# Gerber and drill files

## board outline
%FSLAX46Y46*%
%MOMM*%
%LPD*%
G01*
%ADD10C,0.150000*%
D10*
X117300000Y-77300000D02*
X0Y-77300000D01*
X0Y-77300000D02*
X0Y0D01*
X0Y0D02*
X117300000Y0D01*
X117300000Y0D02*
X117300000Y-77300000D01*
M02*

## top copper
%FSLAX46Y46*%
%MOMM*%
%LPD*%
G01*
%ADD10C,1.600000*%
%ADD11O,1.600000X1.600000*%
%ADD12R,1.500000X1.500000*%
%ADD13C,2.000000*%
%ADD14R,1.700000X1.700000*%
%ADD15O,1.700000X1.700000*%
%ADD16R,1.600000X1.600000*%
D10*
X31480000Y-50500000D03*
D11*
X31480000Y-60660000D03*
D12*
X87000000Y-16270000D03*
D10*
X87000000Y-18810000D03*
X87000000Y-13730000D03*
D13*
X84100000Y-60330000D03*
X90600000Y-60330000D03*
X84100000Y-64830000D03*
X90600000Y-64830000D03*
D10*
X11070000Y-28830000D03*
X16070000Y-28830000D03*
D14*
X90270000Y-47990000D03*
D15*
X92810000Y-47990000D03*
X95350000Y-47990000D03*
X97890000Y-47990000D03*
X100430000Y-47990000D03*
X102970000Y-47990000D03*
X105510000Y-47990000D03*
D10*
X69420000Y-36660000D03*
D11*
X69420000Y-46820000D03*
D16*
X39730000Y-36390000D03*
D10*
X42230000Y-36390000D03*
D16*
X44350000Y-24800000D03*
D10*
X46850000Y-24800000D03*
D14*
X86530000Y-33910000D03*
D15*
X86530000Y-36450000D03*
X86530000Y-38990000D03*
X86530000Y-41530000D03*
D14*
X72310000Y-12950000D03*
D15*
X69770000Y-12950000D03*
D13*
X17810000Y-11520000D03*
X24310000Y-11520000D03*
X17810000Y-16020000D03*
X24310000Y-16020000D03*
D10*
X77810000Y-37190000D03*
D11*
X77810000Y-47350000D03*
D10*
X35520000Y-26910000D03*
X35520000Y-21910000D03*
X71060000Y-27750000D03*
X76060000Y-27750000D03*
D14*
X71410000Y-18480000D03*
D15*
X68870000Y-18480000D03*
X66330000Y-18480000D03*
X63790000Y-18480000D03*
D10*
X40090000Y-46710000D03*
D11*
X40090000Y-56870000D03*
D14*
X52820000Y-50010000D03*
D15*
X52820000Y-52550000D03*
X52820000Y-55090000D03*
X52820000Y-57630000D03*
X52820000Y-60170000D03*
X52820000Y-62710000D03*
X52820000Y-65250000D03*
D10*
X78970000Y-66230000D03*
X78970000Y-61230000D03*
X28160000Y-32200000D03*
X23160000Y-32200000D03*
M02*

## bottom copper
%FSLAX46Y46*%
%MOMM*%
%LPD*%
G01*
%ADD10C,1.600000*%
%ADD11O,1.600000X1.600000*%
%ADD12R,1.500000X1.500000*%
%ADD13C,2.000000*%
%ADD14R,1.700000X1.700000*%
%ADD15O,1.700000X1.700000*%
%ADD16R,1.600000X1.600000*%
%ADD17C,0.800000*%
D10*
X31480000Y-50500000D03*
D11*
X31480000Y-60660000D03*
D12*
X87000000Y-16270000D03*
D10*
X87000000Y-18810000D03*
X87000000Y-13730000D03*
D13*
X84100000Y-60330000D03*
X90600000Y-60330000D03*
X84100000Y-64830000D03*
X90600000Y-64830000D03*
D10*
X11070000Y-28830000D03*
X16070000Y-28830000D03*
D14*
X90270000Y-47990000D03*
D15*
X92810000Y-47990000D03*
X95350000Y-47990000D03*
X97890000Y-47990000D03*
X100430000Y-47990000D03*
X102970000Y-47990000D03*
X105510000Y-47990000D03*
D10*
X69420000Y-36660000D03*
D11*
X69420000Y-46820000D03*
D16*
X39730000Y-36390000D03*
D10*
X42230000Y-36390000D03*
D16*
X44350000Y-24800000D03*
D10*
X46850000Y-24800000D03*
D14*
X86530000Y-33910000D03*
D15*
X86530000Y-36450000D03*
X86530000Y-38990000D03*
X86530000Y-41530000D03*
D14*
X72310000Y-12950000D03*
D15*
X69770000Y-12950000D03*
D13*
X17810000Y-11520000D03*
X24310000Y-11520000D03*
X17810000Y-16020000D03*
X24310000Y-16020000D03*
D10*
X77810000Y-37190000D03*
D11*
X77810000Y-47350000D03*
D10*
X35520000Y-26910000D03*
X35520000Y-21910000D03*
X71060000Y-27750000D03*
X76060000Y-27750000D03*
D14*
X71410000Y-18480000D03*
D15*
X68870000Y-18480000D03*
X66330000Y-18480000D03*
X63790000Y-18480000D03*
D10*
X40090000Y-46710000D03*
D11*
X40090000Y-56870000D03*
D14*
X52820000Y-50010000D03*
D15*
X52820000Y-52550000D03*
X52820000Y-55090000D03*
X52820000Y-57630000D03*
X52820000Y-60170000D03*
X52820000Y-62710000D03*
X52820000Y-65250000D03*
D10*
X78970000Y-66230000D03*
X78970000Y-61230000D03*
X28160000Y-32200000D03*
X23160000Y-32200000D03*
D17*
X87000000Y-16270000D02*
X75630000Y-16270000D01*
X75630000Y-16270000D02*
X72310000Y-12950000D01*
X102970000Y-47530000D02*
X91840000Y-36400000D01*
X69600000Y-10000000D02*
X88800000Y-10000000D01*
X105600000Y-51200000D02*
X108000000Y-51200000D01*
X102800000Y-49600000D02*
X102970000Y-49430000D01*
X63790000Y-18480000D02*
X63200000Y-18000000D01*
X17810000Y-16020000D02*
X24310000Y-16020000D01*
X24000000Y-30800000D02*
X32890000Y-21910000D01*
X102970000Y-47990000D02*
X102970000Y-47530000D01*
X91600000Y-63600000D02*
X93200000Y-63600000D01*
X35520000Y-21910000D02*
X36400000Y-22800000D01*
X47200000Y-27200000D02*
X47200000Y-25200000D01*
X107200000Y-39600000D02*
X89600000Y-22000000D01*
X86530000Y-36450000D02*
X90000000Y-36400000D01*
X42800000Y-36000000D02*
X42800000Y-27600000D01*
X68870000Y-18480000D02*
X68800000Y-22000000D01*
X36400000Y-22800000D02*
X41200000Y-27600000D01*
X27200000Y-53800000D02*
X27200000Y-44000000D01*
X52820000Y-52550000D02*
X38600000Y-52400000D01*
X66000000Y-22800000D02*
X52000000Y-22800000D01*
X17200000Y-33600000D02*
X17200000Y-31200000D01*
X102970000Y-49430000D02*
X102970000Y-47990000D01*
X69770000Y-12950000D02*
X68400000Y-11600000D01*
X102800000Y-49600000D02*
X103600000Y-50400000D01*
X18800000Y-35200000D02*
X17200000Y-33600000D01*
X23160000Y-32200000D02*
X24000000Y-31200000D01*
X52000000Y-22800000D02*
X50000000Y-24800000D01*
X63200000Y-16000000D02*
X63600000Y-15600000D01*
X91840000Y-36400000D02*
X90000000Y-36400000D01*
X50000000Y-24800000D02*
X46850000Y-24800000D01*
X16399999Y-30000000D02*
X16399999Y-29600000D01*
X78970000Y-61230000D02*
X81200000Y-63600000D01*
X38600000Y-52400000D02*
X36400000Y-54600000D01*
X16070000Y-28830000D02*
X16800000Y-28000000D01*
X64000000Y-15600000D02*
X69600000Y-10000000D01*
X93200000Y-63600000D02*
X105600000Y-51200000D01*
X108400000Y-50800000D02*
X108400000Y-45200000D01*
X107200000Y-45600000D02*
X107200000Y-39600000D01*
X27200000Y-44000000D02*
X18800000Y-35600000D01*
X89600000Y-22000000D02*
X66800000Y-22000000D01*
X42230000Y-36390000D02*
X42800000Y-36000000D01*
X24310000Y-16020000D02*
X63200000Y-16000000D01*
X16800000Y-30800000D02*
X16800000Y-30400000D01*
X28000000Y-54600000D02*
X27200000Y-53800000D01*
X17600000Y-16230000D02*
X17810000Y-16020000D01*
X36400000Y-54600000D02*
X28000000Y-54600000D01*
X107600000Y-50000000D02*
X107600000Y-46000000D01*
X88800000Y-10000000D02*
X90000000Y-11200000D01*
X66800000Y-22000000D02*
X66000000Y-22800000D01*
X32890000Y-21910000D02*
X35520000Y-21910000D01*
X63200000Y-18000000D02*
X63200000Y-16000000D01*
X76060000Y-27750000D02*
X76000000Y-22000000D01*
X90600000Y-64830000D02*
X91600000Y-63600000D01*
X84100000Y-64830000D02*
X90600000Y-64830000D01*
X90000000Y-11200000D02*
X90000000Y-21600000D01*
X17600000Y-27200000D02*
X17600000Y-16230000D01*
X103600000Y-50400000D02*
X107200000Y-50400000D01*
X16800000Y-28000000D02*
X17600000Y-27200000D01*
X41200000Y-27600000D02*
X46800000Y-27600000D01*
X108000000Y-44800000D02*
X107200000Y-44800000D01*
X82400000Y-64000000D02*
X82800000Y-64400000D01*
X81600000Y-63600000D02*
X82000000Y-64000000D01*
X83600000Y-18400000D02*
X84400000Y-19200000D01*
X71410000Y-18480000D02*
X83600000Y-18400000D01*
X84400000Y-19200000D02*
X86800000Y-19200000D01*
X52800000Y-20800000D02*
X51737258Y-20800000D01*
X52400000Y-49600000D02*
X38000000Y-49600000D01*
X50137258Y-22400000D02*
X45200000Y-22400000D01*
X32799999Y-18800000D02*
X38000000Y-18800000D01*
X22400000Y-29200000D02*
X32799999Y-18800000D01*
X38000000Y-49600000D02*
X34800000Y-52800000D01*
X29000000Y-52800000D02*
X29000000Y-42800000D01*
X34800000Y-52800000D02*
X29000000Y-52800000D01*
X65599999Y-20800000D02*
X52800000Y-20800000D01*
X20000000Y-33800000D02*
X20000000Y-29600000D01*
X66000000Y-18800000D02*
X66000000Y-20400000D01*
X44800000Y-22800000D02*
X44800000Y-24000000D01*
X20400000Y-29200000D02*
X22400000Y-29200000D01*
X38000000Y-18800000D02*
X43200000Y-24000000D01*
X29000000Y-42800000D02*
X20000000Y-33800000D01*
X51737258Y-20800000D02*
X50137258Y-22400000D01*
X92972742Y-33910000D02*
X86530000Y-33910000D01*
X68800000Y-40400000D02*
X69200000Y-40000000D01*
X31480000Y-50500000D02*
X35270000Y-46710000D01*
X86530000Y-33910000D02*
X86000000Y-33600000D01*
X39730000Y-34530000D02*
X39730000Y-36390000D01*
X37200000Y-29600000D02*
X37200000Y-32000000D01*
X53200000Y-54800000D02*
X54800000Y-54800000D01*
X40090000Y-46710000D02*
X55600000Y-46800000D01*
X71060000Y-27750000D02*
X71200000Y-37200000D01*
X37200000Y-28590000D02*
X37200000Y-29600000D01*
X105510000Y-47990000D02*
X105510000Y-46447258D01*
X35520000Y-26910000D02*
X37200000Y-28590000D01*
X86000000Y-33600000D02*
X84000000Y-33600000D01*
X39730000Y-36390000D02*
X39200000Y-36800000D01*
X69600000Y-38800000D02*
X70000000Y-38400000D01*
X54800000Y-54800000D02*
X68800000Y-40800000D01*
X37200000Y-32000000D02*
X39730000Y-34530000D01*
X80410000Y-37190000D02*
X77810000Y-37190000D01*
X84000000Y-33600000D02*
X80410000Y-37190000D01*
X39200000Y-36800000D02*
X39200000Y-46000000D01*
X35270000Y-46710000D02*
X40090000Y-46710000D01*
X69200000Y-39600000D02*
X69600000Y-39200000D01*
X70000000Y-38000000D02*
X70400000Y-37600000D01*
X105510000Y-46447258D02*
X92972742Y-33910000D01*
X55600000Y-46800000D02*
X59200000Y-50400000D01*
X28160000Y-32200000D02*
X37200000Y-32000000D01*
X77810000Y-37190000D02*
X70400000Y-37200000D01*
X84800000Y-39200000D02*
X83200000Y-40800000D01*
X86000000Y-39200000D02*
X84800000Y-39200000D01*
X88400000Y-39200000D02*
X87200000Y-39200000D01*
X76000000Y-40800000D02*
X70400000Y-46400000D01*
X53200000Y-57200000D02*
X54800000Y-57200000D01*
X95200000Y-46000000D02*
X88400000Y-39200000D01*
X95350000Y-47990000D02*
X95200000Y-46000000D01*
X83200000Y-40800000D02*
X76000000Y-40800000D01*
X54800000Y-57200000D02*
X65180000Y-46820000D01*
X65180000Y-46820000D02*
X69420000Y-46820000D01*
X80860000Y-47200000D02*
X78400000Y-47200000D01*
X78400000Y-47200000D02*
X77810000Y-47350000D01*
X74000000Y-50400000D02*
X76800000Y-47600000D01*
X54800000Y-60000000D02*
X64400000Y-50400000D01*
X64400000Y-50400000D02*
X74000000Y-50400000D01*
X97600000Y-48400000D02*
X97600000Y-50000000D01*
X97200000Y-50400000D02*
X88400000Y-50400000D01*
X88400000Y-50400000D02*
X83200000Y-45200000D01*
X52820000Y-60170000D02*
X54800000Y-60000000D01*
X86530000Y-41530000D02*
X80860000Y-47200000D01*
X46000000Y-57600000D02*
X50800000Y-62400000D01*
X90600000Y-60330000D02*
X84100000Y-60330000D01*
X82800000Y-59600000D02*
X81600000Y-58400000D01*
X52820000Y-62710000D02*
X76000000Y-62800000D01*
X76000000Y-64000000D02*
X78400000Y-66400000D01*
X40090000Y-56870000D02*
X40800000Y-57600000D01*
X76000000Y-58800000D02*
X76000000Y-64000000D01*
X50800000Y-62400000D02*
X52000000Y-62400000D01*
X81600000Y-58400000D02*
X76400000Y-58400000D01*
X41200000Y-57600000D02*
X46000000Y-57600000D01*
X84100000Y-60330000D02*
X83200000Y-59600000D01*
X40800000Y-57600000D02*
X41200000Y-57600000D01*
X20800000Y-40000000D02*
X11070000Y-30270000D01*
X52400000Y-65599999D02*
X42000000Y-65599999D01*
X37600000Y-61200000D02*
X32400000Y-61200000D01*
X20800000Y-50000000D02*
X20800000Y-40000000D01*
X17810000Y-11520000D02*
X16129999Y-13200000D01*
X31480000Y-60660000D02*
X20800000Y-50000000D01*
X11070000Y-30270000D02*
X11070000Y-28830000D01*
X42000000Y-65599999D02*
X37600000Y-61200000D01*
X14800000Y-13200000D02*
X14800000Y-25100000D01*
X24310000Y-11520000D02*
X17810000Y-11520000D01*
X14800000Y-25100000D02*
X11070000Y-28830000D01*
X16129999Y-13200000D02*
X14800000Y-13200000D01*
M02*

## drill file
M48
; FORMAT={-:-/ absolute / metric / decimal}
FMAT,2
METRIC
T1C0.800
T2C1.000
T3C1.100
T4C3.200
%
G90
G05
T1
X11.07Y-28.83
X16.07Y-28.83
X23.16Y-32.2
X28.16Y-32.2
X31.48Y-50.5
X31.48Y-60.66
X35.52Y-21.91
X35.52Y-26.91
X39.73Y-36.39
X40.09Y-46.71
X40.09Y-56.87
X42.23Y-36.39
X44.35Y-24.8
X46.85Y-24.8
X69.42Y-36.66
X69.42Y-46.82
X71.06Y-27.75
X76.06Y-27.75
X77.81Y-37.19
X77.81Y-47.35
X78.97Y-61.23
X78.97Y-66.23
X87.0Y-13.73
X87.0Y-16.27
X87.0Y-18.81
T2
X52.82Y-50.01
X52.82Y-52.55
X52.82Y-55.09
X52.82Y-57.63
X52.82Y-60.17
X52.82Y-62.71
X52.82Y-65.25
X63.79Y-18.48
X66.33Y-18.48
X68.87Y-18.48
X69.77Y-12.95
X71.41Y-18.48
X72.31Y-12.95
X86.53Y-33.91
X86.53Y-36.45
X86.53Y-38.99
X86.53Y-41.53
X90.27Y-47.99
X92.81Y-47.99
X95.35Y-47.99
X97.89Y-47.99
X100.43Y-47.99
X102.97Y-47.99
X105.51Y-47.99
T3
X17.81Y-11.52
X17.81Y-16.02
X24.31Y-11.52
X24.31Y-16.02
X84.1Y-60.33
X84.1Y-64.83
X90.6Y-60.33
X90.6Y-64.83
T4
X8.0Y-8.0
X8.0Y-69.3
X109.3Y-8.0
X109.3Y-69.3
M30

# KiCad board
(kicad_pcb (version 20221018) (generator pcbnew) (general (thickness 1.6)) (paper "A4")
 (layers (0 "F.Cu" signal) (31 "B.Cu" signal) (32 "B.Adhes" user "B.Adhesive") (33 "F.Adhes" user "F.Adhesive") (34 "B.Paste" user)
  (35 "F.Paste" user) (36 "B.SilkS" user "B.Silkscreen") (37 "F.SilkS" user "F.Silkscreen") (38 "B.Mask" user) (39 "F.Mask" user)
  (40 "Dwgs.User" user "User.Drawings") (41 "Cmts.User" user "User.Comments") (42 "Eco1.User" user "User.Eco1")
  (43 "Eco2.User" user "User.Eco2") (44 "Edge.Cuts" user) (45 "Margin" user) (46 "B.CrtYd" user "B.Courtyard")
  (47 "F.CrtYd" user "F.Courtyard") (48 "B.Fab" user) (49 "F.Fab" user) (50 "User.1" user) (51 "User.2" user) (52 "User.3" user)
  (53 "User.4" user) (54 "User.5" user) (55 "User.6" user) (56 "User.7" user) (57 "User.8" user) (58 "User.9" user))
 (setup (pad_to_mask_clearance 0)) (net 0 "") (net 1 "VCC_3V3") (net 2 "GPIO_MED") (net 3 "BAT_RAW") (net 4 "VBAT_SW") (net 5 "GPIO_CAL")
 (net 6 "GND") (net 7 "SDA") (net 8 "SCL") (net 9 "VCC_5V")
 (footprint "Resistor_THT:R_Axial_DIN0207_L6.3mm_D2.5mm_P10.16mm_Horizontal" (layer "F.Cu") (at 31.48 50.5 -90)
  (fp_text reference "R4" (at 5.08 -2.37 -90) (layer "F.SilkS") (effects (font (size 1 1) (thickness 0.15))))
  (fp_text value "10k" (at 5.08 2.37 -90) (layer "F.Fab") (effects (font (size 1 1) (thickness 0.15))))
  (pad "1" thru_hole circle (at 0 0 270) (size 1.6 1.6) (drill 0.8) (layers "*.Cu" "*.Mask") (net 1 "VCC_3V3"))
  (pad "2" thru_hole oval (at 10.16 0 270) (size 1.6 1.6) (drill 0.8) (layers "*.Cu" "*.Mask") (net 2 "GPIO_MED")))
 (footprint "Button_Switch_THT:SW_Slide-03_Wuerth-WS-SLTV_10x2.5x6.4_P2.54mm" (layer "F.Cu") (at 87 16.27 90)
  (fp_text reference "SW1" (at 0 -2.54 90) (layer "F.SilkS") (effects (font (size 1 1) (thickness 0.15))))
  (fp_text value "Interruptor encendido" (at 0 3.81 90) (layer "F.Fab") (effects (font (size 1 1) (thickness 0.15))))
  (pad "1" thru_hole rect (at 0 0 90) (size 1.5 1.5) (drill 0.8) (layers "*.Cu" "*.Mask") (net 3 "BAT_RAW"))
  (pad "2" thru_hole circle (at -2.54 0 90) (size 1.6 1.6) (drill 0.8) (layers "*.Cu" "*.Mask") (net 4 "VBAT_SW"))
  (pad "3" thru_hole circle (at 2.54 0 90) (size 1.6 1.6) (drill 0.8) (layers "*.Cu" "*.Mask")))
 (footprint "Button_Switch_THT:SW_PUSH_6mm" (layer "F.Cu") (at 84.1 60.33)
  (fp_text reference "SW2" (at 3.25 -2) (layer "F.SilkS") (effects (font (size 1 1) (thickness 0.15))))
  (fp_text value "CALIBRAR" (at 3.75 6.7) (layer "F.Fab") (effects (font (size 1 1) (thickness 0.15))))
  (pad "1" thru_hole circle (at 0 0 90) (size 2 2) (drill 1.1) (layers "*.Cu" "*.Mask") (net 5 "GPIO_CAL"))
  (pad "1" thru_hole circle (at 6.5 0 90) (size 2 2) (drill 1.1) (layers "*.Cu" "*.Mask") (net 5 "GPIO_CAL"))
  (pad "2" thru_hole circle (at 0 4.5 90) (size 2 2) (drill 1.1) (layers "*.Cu" "*.Mask") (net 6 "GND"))
  (pad "2" thru_hole circle (at 6.5 4.5 90) (size 2 2) (drill 1.1) (layers "*.Cu" "*.Mask") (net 6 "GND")))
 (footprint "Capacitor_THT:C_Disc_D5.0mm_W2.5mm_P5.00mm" (layer "F.Cu") (at 11.07 28.83)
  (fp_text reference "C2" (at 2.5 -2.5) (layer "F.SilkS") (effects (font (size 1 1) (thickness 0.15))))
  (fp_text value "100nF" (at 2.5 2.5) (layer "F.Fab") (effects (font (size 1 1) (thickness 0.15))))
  (pad "1" thru_hole circle (at 0 0) (size 1.6 1.6) (drill 0.8) (layers "*.Cu" "*.Mask") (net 2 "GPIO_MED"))
  (pad "2" thru_hole circle (at 5 0) (size 1.6 1.6) (drill 0.8) (layers "*.Cu" "*.Mask") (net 6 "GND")))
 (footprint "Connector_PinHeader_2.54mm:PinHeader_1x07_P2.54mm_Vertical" (layer "F.Cu") (at 90.27 47.99 90)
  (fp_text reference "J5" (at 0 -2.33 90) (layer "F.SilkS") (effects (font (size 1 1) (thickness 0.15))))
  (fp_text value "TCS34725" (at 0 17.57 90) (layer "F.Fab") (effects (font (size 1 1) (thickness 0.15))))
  (pad "1" thru_hole rect (at 0 0 90) (size 1.7 1.7) (drill 1) (layers "*.Cu" "*.Mask"))
  (pad "2" thru_hole oval (at 0 2.54 90) (size 1.7 1.7) (drill 1) (layers "*.Cu" "*.Mask"))
  (pad "3" thru_hole oval (at 0 5.08 90) (size 1.7 1.7) (drill 1) (layers "*.Cu" "*.Mask") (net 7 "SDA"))
  (pad "4" thru_hole oval (at 0 7.62 90) (size 1.7 1.7) (drill 1) (layers "*.Cu" "*.Mask") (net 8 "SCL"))
  (pad "5" thru_hole oval (at 0 10.16 90) (size 1.7 1.7) (drill 1) (layers "*.Cu" "*.Mask"))
  (pad "6" thru_hole oval (at 0 12.7 90) (size 1.7 1.7) (drill 1) (layers "*.Cu" "*.Mask") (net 6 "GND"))
  (pad "7" thru_hole oval (at 0 15.24 90) (size 1.7 1.7) (drill 1) (layers "*.Cu" "*.Mask") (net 1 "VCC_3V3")))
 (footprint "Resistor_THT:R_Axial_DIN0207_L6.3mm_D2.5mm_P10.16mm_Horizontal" (layer "F.Cu") (at 69.42 36.66 -90)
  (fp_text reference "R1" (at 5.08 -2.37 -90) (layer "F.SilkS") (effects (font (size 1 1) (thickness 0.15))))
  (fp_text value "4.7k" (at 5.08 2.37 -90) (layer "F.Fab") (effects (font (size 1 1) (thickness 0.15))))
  (pad "1" thru_hole circle (at 0 0 270) (size 1.6 1.6) (drill 0.8) (layers "*.Cu" "*.Mask") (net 1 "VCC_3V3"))
  (pad "2" thru_hole oval (at 10.16 0 270) (size 1.6 1.6) (drill 0.8) (layers "*.Cu" "*.Mask") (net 7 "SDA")))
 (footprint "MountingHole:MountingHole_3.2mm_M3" (layer "F.Cu") (at 8 69.3)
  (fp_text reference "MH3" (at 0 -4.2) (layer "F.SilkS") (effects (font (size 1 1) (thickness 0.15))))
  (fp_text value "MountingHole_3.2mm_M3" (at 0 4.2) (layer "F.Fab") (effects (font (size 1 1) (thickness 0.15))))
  (pad "" np_thru_hole circle (at 0 0) (size 3.2 3.2) (drill 3.2) (layers "*.Cu" "*.Mask")))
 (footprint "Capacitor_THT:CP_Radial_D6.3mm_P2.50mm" (layer "F.Cu") (at 39.73 36.39)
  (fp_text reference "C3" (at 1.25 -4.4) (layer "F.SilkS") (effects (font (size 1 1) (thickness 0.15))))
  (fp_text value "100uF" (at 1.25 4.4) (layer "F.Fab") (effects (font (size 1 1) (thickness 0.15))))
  (pad "1" thru_hole rect (at 0 0) (size 1.6 1.6) (drill 0.8) (layers "*.Cu" "*.Mask") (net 1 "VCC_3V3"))
  (pad "2" thru_hole circle (at 2.5 0) (size 1.6 1.6) (drill 0.8) (layers "*.Cu" "*.Mask") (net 6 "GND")))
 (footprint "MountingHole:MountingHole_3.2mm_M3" (layer "F.Cu") (at 109.3 8)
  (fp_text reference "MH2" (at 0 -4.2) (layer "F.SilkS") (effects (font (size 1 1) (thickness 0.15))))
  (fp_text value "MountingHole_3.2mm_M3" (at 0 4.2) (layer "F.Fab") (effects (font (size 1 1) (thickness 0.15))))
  (pad "" np_thru_hole circle (at 0 0) (size 3.2 3.2) (drill 3.2) (layers "*.Cu" "*.Mask")))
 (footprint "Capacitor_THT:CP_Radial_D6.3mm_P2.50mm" (layer "F.Cu") (at 44.35 24.8)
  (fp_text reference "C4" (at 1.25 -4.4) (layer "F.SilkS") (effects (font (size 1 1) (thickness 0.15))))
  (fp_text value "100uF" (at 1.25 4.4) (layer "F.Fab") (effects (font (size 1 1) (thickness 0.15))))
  (pad "1" thru_hole rect (at 0 0) (size 1.6 1.6) (drill 0.8) (layers "*.Cu" "*.Mask") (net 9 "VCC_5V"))
  (pad "2" thru_hole circle (at 2.5 0) (size 1.6 1.6) (drill 0.8) (layers "*.Cu" "*.Mask") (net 6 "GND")))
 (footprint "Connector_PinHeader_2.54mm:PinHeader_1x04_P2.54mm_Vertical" (layer "F.Cu") (at 86.53 33.91)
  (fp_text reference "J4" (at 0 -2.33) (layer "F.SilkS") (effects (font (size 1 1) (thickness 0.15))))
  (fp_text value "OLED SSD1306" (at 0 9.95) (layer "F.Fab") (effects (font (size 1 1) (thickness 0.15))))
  (pad "1" thru_hole rect (at 0 0) (size 1.7 1.7) (drill 1) (layers "*.Cu" "*.Mask") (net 1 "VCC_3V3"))
  (pad "2" thru_hole oval (at 0 2.54) (size 1.7 1.7) (drill 1) (layers "*.Cu" "*.Mask") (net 6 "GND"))
  (pad "3" thru_hole oval (at 0 5.08) (size 1.7 1.7) (drill 1) (layers "*.Cu" "*.Mask") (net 7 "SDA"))
  (pad "4" thru_hole oval (at 0 7.62) (size 1.7 1.7) (drill 1) (layers "*.Cu" "*.Mask") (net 8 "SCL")))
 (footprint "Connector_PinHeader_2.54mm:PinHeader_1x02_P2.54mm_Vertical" (layer "F.Cu") (at 72.31 12.95 -90)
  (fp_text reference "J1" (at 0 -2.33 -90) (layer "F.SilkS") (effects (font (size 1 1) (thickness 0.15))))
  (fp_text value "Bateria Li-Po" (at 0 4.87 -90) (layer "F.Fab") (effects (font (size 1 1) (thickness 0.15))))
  (pad "1" thru_hole rect (at 0 0 270) (size 1.7 1.7) (drill 1) (layers "*.Cu" "*.Mask") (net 3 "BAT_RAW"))
  (pad "2" thru_hole oval (at 0 2.54 270) (size 1.7 1.7) (drill 1) (layers "*.Cu" "*.Mask") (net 6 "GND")))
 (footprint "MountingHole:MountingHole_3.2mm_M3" (layer "F.Cu") (at 109.3 69.3)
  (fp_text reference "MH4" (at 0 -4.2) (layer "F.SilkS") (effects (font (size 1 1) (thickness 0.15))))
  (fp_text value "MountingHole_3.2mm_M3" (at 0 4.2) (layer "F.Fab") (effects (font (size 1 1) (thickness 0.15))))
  (pad "" np_thru_hole circle (at 0 0) (size 3.2 3.2) (drill 3.2) (layers "*.Cu" "*.Mask")))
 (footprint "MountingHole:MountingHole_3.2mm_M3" (layer "F.Cu") (at 8 8)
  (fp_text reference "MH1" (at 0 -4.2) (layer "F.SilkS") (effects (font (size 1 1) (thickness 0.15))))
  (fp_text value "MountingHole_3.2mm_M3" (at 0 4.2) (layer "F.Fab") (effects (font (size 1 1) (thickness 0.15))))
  (pad "" np_thru_hole circle (at 0 0) (size 3.2 3.2) (drill 3.2) (layers "*.Cu" "*.Mask")))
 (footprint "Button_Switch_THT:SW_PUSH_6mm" (layer "F.Cu") (at 17.81 11.52)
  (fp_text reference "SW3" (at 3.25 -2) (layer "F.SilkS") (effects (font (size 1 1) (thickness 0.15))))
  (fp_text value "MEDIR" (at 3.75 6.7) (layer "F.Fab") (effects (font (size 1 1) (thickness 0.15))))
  (pad "1" thru_hole circle (at 0 0 90) (size 2 2) (drill 1.1) (layers "*.Cu" "*.Mask") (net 2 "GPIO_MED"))
  (pad "1" thru_hole circle (at 6.5 0 90) (size 2 2) (drill 1.1) (layers "*.Cu" "*.Mask") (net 2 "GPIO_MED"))
  (pad "2" thru_hole circle (at 0 4.5 90) (size 2 2) (drill 1.1) (layers "*.Cu" "*.Mask") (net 6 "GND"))
  (pad "2" thru_hole circle (at 6.5 4.5 90) (size 2 2) (drill 1.1) (layers "*.Cu" "*.Mask") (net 6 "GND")))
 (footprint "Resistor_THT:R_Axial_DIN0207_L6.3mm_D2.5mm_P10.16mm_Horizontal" (layer "F.Cu") (at 77.81 37.19 -90)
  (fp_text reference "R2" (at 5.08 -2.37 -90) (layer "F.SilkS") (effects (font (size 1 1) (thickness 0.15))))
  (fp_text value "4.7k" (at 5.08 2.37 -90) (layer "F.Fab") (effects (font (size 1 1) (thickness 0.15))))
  (pad "1" thru_hole circle (at 0 0 270) (size 1.6 1.6) (drill 0.8) (layers "*.Cu" "*.Mask") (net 1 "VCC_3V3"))
  (pad "2" thru_hole oval (at 10.16 0 270) (size 1.6 1.6) (drill 0.8) (layers "*.Cu" "*.Mask") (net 8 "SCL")))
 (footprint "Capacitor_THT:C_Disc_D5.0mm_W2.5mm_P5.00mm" (layer "F.Cu") (at 35.52 26.91 90)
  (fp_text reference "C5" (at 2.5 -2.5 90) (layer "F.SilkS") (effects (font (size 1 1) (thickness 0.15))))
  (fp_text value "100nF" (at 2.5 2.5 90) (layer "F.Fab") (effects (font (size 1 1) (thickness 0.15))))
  (pad "1" thru_hole circle (at 0 0 90) (size 1.6 1.6) (drill 0.8) (layers "*.Cu" "*.Mask") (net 1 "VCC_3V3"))
  (pad "2" thru_hole circle (at 5 0 90) (size 1.6 1.6) (drill 0.8) (layers "*.Cu" "*.Mask") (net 6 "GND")))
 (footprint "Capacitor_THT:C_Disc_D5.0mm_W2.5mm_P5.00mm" (layer "F.Cu") (at 71.06 27.75)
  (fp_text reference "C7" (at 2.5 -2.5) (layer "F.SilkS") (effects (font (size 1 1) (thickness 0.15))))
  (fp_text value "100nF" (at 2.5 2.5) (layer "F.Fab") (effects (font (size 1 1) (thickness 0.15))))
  (pad "1" thru_hole circle (at 0 0) (size 1.6 1.6) (drill 0.8) (layers "*.Cu" "*.Mask") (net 1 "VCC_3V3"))
  (pad "2" thru_hole circle (at 5 0) (size 1.6 1.6) (drill 0.8) (layers "*.Cu" "*.Mask") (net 6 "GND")))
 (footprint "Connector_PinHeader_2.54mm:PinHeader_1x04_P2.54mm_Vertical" (layer "F.Cu") (at 71.41 18.48 -90)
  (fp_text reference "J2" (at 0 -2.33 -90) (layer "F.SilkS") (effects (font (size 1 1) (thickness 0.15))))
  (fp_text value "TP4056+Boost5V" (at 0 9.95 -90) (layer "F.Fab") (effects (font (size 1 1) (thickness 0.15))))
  (pad "1" thru_hole rect (at 0 0 270) (size 1.7 1.7) (drill 1) (layers "*.Cu" "*.Mask") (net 4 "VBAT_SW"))
  (pad "2" thru_hole oval (at 0 2.54 270) (size 1.7 1.7) (drill 1) (layers "*.Cu" "*.Mask") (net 6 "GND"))
  (pad "3" thru_hole oval (at 0 5.08 270) (size 1.7 1.7) (drill 1) (layers "*.Cu" "*.Mask") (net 9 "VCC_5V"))
  (pad "4" thru_hole oval (at 0 7.62 270) (size 1.7 1.7) (drill 1) (layers "*.Cu" "*.Mask") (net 6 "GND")))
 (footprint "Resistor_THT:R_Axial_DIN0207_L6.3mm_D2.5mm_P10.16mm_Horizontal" (layer "F.Cu") (at 40.09 46.71 -90)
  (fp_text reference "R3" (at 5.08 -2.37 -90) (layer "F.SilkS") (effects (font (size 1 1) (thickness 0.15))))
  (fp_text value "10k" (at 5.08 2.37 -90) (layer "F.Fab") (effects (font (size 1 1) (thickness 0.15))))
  (pad "1" thru_hole circle (at 0 0 270) (size 1.6 1.6) (drill 0.8) (layers "*.Cu" "*.Mask") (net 1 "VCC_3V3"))
  (pad "2" thru_hole oval (at 10.16 0 270) (size 1.6 1.6) (drill 0.8) (layers "*.Cu" "*.Mask") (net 5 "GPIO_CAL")))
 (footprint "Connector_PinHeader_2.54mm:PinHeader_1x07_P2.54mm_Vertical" (layer "F.Cu") (at 52.82 50.01)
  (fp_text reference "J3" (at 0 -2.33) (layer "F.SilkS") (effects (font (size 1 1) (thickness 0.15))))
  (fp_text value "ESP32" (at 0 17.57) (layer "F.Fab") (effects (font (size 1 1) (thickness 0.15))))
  (pad "1" thru_hole rect (at 0 0) (size 1.7 1.7) (drill 1) (layers "*.Cu" "*.Mask") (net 9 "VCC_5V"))
  (pad "2" thru_hole oval (at 0 2.54) (size 1.7 1.7) (drill 1) (layers "*.Cu" "*.Mask") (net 6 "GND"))
  (pad "3" thru_hole oval (at 0 5.08) (size 1.7 1.7) (drill 1) (layers "*.Cu" "*.Mask") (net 1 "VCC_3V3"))
  (pad "4" thru_hole oval (at 0 7.62) (size 1.7 1.7) (drill 1) (layers "*.Cu" "*.Mask") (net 7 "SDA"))
  (pad "5" thru_hole oval (at 0 10.16) (size 1.7 1.7) (drill 1) (layers "*.Cu" "*.Mask") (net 8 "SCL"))
  (pad "6" thru_hole oval (at 0 12.7) (size 1.7 1.7) (drill 1) (layers "*.Cu" "*.Mask") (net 5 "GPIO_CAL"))
  (pad "7" thru_hole oval (at 0 15.24) (size 1.7 1.7) (drill 1) (layers "*.Cu" "*.Mask") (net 2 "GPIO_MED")))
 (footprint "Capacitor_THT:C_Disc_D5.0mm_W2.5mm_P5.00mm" (layer "F.Cu") (at 78.97 66.23 90)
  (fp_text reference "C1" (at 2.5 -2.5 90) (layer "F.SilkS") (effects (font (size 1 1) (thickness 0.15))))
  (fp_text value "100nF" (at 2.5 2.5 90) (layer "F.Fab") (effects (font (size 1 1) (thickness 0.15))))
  (pad "1" thru_hole circle (at 0 0 90) (size 1.6 1.6) (drill 0.8) (layers "*.Cu" "*.Mask") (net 5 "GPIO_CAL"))
  (pad "2" thru_hole circle (at 5 0 90) (size 1.6 1.6) (drill 0.8) (layers "*.Cu" "*.Mask") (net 6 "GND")))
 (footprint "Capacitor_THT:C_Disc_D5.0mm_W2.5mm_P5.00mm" (layer "F.Cu") (at 28.16 32.2 180)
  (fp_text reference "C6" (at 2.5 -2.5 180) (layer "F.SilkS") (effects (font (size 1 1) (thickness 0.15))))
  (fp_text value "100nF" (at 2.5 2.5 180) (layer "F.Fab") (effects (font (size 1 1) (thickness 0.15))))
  (pad "1" thru_hole circle (at 0 0 180) (size 1.6 1.6) (drill 0.8) (layers "*.Cu" "*.Mask") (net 1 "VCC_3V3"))
  (pad "2" thru_hole circle (at 5 0 180) (size 1.6 1.6) (drill 0.8) (layers "*.Cu" "*.Mask") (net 6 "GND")))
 (gr_line (start 117.3 77.3) (end 0 77.3) (stroke (width 0.15) (type default)) (layer "Edge.Cuts"))
 (gr_line (start 0 77.3) (end 0 0) (stroke (width 0.15) (type default)) (layer "Edge.Cuts"))
 (gr_line (start 0 0) (end 117.3 0) (stroke (width 0.15) (type default)) (layer "Edge.Cuts"))
 (gr_line (start 117.3 0) (end 117.3 77.3) (stroke (width 0.15) (type default)) (layer "Edge.Cuts"))
 (segment (start 87 16.27) (end 75.63 16.27) (width 0.8) (layer "B.Cu") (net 3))
 (segment (start 75.63 16.27) (end 72.31 12.95) (width 0.8) (layer "B.Cu") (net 3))
 (segment (start 102.97 47.53) (end 91.84 36.4) (width 0.8) (layer "B.Cu") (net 6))
 (segment (start 69.6 10) (end 88.8 10) (width 0.8) (layer "B.Cu") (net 6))
 (segment (start 105.6 51.2) (end 108 51.2) (width 0.8) (layer "B.Cu") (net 6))
 (segment (start 102.8 49.6) (end 102.97 49.43) (width 0.8) (layer "B.Cu") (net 6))
 (segment (start 63.79 18.48) (end 63.2 18) (width 0.8) (layer "B.Cu") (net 6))
 (segment (start 17.81 16.02) (end 24.31 16.02) (width 0.8) (layer "B.Cu") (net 6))
 (segment (start 24 30.8) (end 32.89 21.91) (width 0.8) (layer "B.Cu") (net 6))
 (segment (start 102.97 47.99) (end 102.97 47.53) (width 0.8) (layer "B.Cu") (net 6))
 (segment (start 91.6 63.6) (end 93.2 63.6) (width 0.8) (layer "B.Cu") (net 6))
 (segment (start 35.52 21.91) (end 36.4 22.8) (width 0.8) (layer "B.Cu") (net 6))
 (segment (start 47.2 27.2) (end 47.2 25.2) (width 0.8) (layer "B.Cu") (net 6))
 (segment (start 107.2 39.6) (end 89.6 22) (width 0.8) (layer "B.Cu") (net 6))
 (segment (start 86.53 36.45) (end 90 36.4) (width 0.8) (layer "B.Cu") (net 6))
 (segment (start 42.8 36) (end 42.8 27.6) (width 0.8) (layer "B.Cu") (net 6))
 (segment (start 68.87 18.48) (end 68.8 22) (width 0.8) (layer "B.Cu") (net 6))
 (segment (start 36.4 22.8) (end 41.2 27.6) (width 0.8) (layer "B.Cu") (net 6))
 (segment (start 27.2 53.8) (end 27.2 44) (width 0.8) (layer "B.Cu") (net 6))
 (segment (start 52.82 52.55) (end 38.6 52.4) (width 0.8) (layer "B.Cu") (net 6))
 (segment (start 66 22.8) (end 52 22.8) (width 0.8) (layer "B.Cu") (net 6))
 (segment (start 17.2 33.6) (end 17.2 31.2) (width 0.8) (layer "B.Cu") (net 6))
 (segment (start 102.97 49.43) (end 102.97 47.99) (width 0.8) (layer "B.Cu") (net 6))
 (segment (start 69.77 12.95) (end 68.4 11.6) (width 0.8) (layer "B.Cu") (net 6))
 (segment (start 102.8 49.6) (end 103.6 50.4) (width 0.8) (layer "B.Cu") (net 6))
 (segment (start 18.8 35.2) (end 17.2 33.6) (width 0.8) (layer "B.Cu") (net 6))
 (segment (start 23.16 32.2) (end 24 31.2) (width 0.8) (layer "B.Cu") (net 6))
 (segment (start 52 22.8) (end 50 24.8) (width 0.8) (layer "B.Cu") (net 6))
 (segment (start 63.2 16) (end 63.6 15.6) (width 0.8) (layer "B.Cu") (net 6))
 (segment (start 91.84 36.4) (end 90 36.4) (width 0.8) (layer "B.Cu") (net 6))
 (segment (start 50 24.8) (end 46.85 24.8) (width 0.8) (layer "B.Cu") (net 6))
 (segment (start 16.399999 30) (end 16.399999 29.6) (width 0.8) (layer "B.Cu") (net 6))
 (segment (start 78.97 61.23) (end 81.2 63.6) (width 0.8) (layer "B.Cu") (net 6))
 (segment (start 38.6 52.4) (end 36.4 54.6) (width 0.8) (layer "B.Cu") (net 6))
 (segment (start 16.07 28.83) (end 16.8 28) (width 0.8) (layer "B.Cu") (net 6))
 (segment (start 64 15.6) (end 69.6 10) (width 0.8) (layer "B.Cu") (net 6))
 (segment (start 93.2 63.6) (end 105.6 51.2) (width 0.8) (layer "B.Cu") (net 6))
 (segment (start 108.4 50.8) (end 108.4 45.2) (width 0.8) (layer "B.Cu") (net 6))
 (segment (start 107.2 45.6) (end 107.2 39.6) (width 0.8) (layer "B.Cu") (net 6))
 (segment (start 27.2 44) (end 18.8 35.6) (width 0.8) (layer "B.Cu") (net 6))
 (segment (start 89.6 22) (end 66.8 22) (width 0.8) (layer "B.Cu") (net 6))
 (segment (start 42.23 36.39) (end 42.8 36) (width 0.8) (layer "B.Cu") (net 6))
 (segment (start 24.31 16.02) (end 63.2 16) (width 0.8) (layer "B.Cu") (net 6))
 (segment (start 16.8 30.8) (end 16.8 30.4) (width 0.8) (layer "B.Cu") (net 6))
 (segment (start 28 54.6) (end 27.2 53.8) (width 0.8) (layer "B.Cu") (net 6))
 (segment (start 17.6 16.23) (end 17.81 16.02) (width 0.8) (layer "B.Cu") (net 6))
 (segment (start 36.4 54.6) (end 28 54.6) (width 0.8) (layer "B.Cu") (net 6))
 (segment (start 107.6 50) (end 107.6 46) (width 0.8) (layer "B.Cu") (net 6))
 (segment (start 88.8 10) (end 90 11.2) (width 0.8) (layer "B.Cu") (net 6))
 (segment (start 66.8 22) (end 66 22.8) (width 0.8) (layer "B.Cu") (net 6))
 (segment (start 32.89 21.91) (end 35.52 21.91) (width 0.8) (layer "B.Cu") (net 6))
 (segment (start 63.2 18) (end 63.2 16) (width 0.8) (layer "B.Cu") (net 6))
 (segment (start 76.06 27.75) (end 76 22) (width 0.8) (layer "B.Cu") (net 6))
 (segment (start 90.6 64.83) (end 91.6 63.6) (width 0.8) (layer "B.Cu") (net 6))
 (segment (start 84.1 64.83) (end 90.6 64.83) (width 0.8) (layer "B.Cu") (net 6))
 (segment (start 90 11.2) (end 90 21.6) (width 0.8) (layer "B.Cu") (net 6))
 (segment (start 17.6 27.2) (end 17.6 16.23) (width 0.8) (layer "B.Cu") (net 6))
 (segment (start 103.6 50.4) (end 107.2 50.4) (width 0.8) (layer "B.Cu") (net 6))
 (segment (start 16.8 28) (end 17.6 27.2) (width 0.8) (layer "B.Cu") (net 6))
 (segment (start 41.2 27.6) (end 46.8 27.6) (width 0.8) (layer "B.Cu") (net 6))
 (segment (start 108 44.8) (end 107.2 44.8) (width 0.8) (layer "B.Cu") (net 6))
 (segment (start 82.4 64) (end 82.8 64.4) (width 0.8) (layer "B.Cu") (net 6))
 (segment (start 81.6 63.6) (end 82 64) (width 0.8) (layer "B.Cu") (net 6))
 (segment (start 83.6 18.4) (end 84.4 19.2) (width 0.8) (layer "B.Cu") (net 4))
 (segment (start 71.41 18.48) (end 83.6 18.4) (width 0.8) (layer "B.Cu") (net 4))
 (segment (start 84.4 19.2) (end 86.8 19.2) (width 0.8) (layer "B.Cu") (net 4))
 (segment (start 52.8 20.8) (end 51.737258 20.8) (width 0.8) (layer "B.Cu") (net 9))
 (segment (start 52.4 49.6) (end 38 49.6) (width 0.8) (layer "B.Cu") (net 9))
 (segment (start 50.137258 22.4) (end 45.2 22.4) (width 0.8) (layer "B.Cu") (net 9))
 (segment (start 32.799999 18.8) (end 38 18.8) (width 0.8) (layer "B.Cu") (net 9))
 (segment (start 22.4 29.2) (end 32.799999 18.8) (width 0.8) (layer "B.Cu") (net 9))
 (segment (start 38 49.6) (end 34.8 52.8) (width 0.8) (layer "B.Cu") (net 9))
 (segment (start 29 52.8) (end 29 42.8) (width 0.8) (layer "B.Cu") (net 9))
 (segment (start 34.8 52.8) (end 29 52.8) (width 0.8) (layer "B.Cu") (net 9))
 (segment (start 65.599999 20.8) (end 52.8 20.8) (width 0.8) (layer "B.Cu") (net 9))
 (segment (start 20 33.8) (end 20 29.6) (width 0.8) (layer "B.Cu") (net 9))
 (segment (start 66 18.8) (end 66 20.4) (width 0.8) (layer "B.Cu") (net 9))
 (segment (start 44.8 22.8) (end 44.8 24) (width 0.8) (layer "B.Cu") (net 9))
 (segment (start 20.4 29.2) (end 22.4 29.2) (width 0.8) (layer "B.Cu") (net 9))
 (segment (start 38 18.8) (end 43.2 24) (width 0.8) (layer "B.Cu") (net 9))
 (segment (start 29 42.8) (end 20 33.8) (width 0.8) (layer "B.Cu") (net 9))
 (segment (start 51.737258 20.8) (end 50.137258 22.4) (width 0.8) (layer "B.Cu") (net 9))
 (segment (start 92.972742 33.91) (end 86.53 33.91) (width 0.8) (layer "B.Cu") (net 1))
 (segment (start 68.8 40.4) (end 69.2 40) (width 0.8) (layer "B.Cu") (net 1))
 (segment (start 31.48 50.5) (end 35.27 46.71) (width 0.8) (layer "B.Cu") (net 1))
 (segment (start 86.53 33.91) (end 86 33.6) (width 0.8) (layer "B.Cu") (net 1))
 (segment (start 39.73 34.53) (end 39.73 36.39) (width 0.8) (layer "B.Cu") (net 1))
 (segment (start 37.2 29.6) (end 37.2 32) (width 0.8) (layer "B.Cu") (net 1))
 (segment (start 53.2 54.8) (end 54.8 54.8) (width 0.8) (layer "B.Cu") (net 1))
 (segment (start 40.09 46.71) (end 55.6 46.8) (width 0.8) (layer "B.Cu") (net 1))
 (segment (start 71.06 27.75) (end 71.2 37.2) (width 0.8) (layer "B.Cu") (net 1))
 (segment (start 37.2 28.59) (end 37.2 29.6) (width 0.8) (layer "B.Cu") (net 1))
 (segment (start 105.51 47.99) (end 105.51 46.447258) (width 0.8) (layer "B.Cu") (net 1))
 (segment (start 35.52 26.91) (end 37.2 28.59) (width 0.8) (layer "B.Cu") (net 1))
 (segment (start 86 33.6) (end 84 33.6) (width 0.8) (layer "B.Cu") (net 1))
 (segment (start 39.73 36.39) (end 39.2 36.8) (width 0.8) (layer "B.Cu") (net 1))
 (segment (start 69.6 38.8) (end 70 38.4) (width 0.8) (layer "B.Cu") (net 1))
 (segment (start 54.8 54.8) (end 68.8 40.8) (width 0.8) (layer "B.Cu") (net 1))
 (segment (start 37.2 32) (end 39.73 34.53) (width 0.8) (layer "B.Cu") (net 1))
 (segment (start 80.41 37.19) (end 77.81 37.19) (width 0.8) (layer "B.Cu") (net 1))
 (segment (start 84 33.6) (end 80.41 37.19) (width 0.8) (layer "B.Cu") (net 1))
 (segment (start 39.2 36.8) (end 39.2 46) (width 0.8) (layer "B.Cu") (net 1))
 (segment (start 35.27 46.71) (end 40.09 46.71) (width 0.8) (layer "B.Cu") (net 1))
 (segment (start 69.2 39.6) (end 69.6 39.2) (width 0.8) (layer "B.Cu") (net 1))
 (segment (start 70 38) (end 70.4 37.6) (width 0.8) (layer "B.Cu") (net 1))
 (segment (start 105.51 46.447258) (end 92.972742 33.91) (width 0.8) (layer "B.Cu") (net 1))
 (segment (start 55.6 46.8) (end 59.2 50.4) (width 0.8) (layer "B.Cu") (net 1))
 (segment (start 28.16 32.2) (end 37.2 32) (width 0.8) (layer "B.Cu") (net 1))
 (segment (start 77.81 37.19) (end 70.4 37.2) (width 0.8) (layer "B.Cu") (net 1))
 (segment (start 84.8 39.2) (end 83.2 40.8) (width 0.8) (layer "B.Cu") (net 7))
 (segment (start 86 39.2) (end 84.8 39.2) (width 0.8) (layer "B.Cu") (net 7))
 (segment (start 88.4 39.2) (end 87.2 39.2) (width 0.8) (layer "B.Cu") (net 7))
 (segment (start 76 40.8) (end 70.4 46.4) (width 0.8) (layer "B.Cu") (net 7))
 (segment (start 53.2 57.2) (end 54.8 57.2) (width 0.8) (layer "B.Cu") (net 7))
 (segment (start 95.2 46) (end 88.4 39.2) (width 0.8) (layer "B.Cu") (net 7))
 (segment (start 95.35 47.99) (end 95.2 46) (width 0.8) (layer "B.Cu") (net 7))
 (segment (start 83.2 40.8) (end 76 40.8) (width 0.8) (layer "B.Cu") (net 7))
 (segment (start 54.8 57.2) (end 65.18 46.82) (width 0.8) (layer "B.Cu") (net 7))
 (segment (start 65.18 46.82) (end 69.42 46.82) (width 0.8) (layer "B.Cu") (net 7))
 (segment (start 80.86 47.2) (end 78.4 47.2) (width 0.8) (layer "B.Cu") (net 8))
 (segment (start 78.4 47.2) (end 77.81 47.35) (width 0.8) (layer "B.Cu") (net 8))
 (segment (start 74 50.4) (end 76.8 47.6) (width 0.8) (layer "B.Cu") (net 8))
 (segment (start 54.8 60) (end 64.4 50.4) (width 0.8) (layer "B.Cu") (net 8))
 (segment (start 64.4 50.4) (end 74 50.4) (width 0.8) (layer "B.Cu") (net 8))
 (segment (start 97.6 48.4) (end 97.6 50) (width 0.8) (layer "B.Cu") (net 8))
 (segment (start 97.2 50.4) (end 88.4 50.4) (width 0.8) (layer "B.Cu") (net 8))
 (segment (start 88.4 50.4) (end 83.2 45.2) (width 0.8) (layer "B.Cu") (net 8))
 (segment (start 52.82 60.17) (end 54.8 60) (width 0.8) (layer "B.Cu") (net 8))
 (segment (start 86.53 41.53) (end 80.86 47.2) (width 0.8) (layer "B.Cu") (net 8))
 (segment (start 46 57.6) (end 50.8 62.4) (width 0.8) (layer "B.Cu") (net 5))
 (segment (start 90.6 60.33) (end 84.1 60.33) (width 0.8) (layer "B.Cu") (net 5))
 (segment (start 82.8 59.6) (end 81.6 58.4) (width 0.8) (layer "B.Cu") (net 5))
 (segment (start 52.82 62.71) (end 76 62.8) (width 0.8) (layer "B.Cu") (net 5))
 (segment (start 76 64) (end 78.4 66.4) (width 0.8) (layer "B.Cu") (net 5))
 (segment (start 40.09 56.87) (end 40.8 57.6) (width 0.8) (layer "B.Cu") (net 5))
 (segment (start 76 58.8) (end 76 64) (width 0.8) (layer "B.Cu") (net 5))
 (segment (start 50.8 62.4) (end 52 62.4) (width 0.8) (layer "B.Cu") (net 5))
 (segment (start 81.6 58.4) (end 76.4 58.4) (width 0.8) (layer "B.Cu") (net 5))
 (segment (start 41.2 57.6) (end 46 57.6) (width 0.8) (layer "B.Cu") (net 5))
 (segment (start 84.1 60.33) (end 83.2 59.6) (width 0.8) (layer "B.Cu") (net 5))
 (segment (start 40.8 57.6) (end 41.2 57.6) (width 0.8) (layer "B.Cu") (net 5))
 (segment (start 20.8 40) (end 11.07 30.27) (width 0.8) (layer "B.Cu") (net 2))
 (segment (start 52.4 65.599999) (end 42 65.599999) (width 0.8) (layer "B.Cu") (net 2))
 (segment (start 37.6 61.2) (end 32.4 61.2) (width 0.8) (layer "B.Cu") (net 2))
 (segment (start 20.8 50) (end 20.8 40) (width 0.8) (layer "B.Cu") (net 2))
 (segment (start 17.81 11.52) (end 16.129999 13.2) (width 0.8) (layer "B.Cu") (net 2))
 (segment (start 31.48 60.66) (end 20.8 50) (width 0.8) (layer "B.Cu") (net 2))
 (segment (start 11.07 30.27) (end 11.07 28.83) (width 0.8) (layer "B.Cu") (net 2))
 (segment (start 42 65.599999) (end 37.6 61.2) (width 0.8) (layer "B.Cu") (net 2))
 (segment (start 14.8 13.2) (end 14.8 25.1) (width 0.8) (layer "B.Cu") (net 2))
 (segment (start 24.31 11.52) (end 17.81 11.52) (width 0.8) (layer "B.Cu") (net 2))
 (segment (start 14.8 25.1) (end 11.07 28.83) (width 0.8) (layer "B.Cu") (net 2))
 (segment (start 16.129999 13.2) (end 14.8 13.2) (width 0.8) (layer "B.Cu") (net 2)))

